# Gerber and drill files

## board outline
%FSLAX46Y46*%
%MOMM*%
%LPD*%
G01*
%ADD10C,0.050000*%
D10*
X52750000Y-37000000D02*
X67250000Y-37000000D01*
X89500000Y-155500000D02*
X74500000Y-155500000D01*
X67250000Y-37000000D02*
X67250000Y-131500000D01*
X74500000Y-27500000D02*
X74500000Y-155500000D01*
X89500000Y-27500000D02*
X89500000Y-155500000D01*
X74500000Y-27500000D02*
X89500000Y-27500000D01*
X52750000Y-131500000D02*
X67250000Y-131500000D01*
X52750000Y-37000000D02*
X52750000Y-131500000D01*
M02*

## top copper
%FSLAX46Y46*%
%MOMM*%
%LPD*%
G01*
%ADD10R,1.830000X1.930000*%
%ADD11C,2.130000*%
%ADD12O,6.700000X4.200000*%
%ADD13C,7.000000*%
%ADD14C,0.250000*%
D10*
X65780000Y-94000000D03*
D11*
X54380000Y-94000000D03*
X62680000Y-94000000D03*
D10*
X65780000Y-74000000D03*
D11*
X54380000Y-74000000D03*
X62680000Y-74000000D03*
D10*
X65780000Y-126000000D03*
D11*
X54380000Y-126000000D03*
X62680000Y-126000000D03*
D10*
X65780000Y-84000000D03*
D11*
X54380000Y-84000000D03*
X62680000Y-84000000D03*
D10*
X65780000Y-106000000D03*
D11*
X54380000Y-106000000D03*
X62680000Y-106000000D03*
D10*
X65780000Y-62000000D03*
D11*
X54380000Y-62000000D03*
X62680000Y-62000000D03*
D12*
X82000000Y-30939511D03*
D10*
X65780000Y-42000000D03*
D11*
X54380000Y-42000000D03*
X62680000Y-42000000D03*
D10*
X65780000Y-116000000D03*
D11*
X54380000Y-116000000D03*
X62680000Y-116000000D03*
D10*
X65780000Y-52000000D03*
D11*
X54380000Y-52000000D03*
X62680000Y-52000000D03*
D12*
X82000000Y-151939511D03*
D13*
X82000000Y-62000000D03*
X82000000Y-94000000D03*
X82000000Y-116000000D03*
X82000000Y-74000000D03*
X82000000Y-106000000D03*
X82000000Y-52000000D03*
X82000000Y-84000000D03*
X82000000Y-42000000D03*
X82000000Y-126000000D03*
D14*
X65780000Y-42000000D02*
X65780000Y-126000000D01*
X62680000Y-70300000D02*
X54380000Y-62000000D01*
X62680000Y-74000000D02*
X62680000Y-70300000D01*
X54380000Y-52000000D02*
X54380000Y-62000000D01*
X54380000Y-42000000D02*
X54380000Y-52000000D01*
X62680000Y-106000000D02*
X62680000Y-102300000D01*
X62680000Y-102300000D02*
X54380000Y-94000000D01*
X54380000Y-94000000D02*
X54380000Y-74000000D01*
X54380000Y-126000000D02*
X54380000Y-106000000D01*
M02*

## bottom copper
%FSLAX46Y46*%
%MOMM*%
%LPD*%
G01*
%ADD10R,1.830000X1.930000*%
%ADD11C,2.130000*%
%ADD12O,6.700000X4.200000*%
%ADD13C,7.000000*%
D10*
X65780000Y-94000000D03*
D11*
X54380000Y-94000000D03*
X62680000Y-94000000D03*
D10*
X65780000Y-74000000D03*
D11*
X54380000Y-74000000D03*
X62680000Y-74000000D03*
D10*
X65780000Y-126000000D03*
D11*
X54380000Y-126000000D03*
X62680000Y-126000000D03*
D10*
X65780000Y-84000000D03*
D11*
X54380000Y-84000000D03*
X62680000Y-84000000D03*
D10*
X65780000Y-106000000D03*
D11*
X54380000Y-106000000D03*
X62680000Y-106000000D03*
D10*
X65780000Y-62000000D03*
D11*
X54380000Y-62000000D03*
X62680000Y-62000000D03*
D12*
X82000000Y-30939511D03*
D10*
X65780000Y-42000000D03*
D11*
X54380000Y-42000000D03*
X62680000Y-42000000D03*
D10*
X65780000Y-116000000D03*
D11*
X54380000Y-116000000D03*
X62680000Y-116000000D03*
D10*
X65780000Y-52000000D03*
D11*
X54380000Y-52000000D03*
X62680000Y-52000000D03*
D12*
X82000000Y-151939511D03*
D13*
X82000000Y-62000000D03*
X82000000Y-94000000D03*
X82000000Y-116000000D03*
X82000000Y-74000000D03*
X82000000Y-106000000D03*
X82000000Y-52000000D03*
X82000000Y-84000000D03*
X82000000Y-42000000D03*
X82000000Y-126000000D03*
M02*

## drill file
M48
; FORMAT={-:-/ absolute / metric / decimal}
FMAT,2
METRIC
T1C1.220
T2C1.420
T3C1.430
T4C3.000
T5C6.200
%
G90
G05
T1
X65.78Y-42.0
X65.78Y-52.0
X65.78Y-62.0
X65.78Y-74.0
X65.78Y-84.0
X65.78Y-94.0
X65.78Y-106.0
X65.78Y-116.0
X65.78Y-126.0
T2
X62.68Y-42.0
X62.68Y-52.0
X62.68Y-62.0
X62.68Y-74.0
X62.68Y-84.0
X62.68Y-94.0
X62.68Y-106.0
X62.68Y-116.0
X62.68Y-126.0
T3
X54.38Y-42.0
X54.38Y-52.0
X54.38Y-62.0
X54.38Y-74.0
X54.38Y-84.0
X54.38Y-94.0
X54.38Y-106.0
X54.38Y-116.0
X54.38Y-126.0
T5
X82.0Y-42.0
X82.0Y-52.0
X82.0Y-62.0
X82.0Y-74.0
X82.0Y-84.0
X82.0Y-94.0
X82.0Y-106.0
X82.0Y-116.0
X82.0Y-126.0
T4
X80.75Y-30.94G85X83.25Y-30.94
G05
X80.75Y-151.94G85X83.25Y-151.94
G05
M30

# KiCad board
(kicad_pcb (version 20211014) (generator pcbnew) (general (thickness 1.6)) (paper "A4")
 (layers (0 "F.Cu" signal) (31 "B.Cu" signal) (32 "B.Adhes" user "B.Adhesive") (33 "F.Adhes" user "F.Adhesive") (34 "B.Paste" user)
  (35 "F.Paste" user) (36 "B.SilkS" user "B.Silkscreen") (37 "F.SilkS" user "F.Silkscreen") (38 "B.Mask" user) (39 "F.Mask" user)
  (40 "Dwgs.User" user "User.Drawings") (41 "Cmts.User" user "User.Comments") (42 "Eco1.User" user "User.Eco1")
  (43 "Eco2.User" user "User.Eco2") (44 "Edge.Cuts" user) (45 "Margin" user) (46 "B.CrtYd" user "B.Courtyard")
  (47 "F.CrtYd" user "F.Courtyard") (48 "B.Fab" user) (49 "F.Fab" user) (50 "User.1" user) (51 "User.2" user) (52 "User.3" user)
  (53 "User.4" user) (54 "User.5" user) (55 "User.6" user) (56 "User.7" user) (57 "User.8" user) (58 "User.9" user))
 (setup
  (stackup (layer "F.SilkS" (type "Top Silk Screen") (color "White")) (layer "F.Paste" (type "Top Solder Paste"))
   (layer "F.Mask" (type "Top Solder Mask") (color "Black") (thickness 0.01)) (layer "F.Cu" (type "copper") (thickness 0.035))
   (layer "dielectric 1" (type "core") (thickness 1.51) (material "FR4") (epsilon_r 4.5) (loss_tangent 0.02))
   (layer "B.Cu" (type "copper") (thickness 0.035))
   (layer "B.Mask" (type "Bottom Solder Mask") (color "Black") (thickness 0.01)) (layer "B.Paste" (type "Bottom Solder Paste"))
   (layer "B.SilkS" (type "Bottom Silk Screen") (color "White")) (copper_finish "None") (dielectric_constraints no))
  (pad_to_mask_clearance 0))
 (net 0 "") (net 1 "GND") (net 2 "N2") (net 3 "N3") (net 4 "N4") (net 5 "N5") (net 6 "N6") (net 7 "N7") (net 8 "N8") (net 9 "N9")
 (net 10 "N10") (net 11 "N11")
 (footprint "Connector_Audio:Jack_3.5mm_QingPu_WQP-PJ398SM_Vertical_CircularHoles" (layer "F.Cu") (at 65.78 94 -90)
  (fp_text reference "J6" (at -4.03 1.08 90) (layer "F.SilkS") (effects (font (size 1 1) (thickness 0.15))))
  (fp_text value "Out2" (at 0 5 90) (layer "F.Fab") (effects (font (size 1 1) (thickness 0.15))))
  (pad "S" thru_hole rect locked (at 0 0 90) (size 1.93 1.83) (drill 1.22) (layers *.Cu *.Mask) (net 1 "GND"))
  (pad "T" thru_hole circle locked (at 0 11.4 90) (size 2.13 2.13) (drill 1.43) (layers *.Cu *.Mask) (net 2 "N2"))
  (pad "TN" thru_hole circle locked (at 0 3.1 90) (size 2.13 2.13) (drill 1.42) (layers *.Cu *.Mask) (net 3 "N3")))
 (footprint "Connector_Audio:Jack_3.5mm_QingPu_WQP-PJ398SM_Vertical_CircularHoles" (layer "F.Cu") (at 65.78 74 -90)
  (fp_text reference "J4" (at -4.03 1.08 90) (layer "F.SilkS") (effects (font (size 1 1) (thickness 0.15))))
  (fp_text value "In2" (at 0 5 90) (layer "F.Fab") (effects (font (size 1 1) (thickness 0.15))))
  (pad "S" thru_hole rect locked (at 0 0 90) (size 1.93 1.83) (drill 1.22) (layers *.Cu *.Mask) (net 1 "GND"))
  (pad "T" thru_hole circle locked (at 0 11.4 90) (size 2.13 2.13) (drill 1.43) (layers *.Cu *.Mask) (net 2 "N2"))
  (pad "TN" thru_hole circle locked (at 0 3.1 90) (size 2.13 2.13) (drill 1.42) (layers *.Cu *.Mask) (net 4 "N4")))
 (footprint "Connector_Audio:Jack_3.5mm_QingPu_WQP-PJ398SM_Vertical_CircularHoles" (layer "F.Cu") (at 65.78 126 -90)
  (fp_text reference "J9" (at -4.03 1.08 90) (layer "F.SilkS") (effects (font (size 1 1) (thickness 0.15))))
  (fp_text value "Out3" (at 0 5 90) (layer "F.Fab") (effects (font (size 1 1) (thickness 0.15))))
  (pad "S" thru_hole rect locked (at 0 0 90) (size 1.93 1.83) (drill 1.22) (layers *.Cu *.Mask) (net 1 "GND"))
  (pad "T" thru_hole circle locked (at 0 11.4 90) (size 2.13 2.13) (drill 1.43) (layers *.Cu *.Mask) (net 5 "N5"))
  (pad "TN" thru_hole circle locked (at 0 3.1 90) (size 2.13 2.13) (drill 1.42) (layers *.Cu *.Mask) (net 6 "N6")))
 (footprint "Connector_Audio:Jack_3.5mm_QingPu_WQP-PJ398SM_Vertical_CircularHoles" (layer "F.Cu") (at 65.78 84 -90)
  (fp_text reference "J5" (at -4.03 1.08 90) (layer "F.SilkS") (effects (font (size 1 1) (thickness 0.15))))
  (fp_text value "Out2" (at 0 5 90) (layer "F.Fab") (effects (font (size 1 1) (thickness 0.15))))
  (pad "S" thru_hole rect locked (at 0 0 90) (size 1.93 1.83) (drill 1.22) (layers *.Cu *.Mask) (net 1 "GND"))
  (pad "T" thru_hole circle locked (at 0 11.4 90) (size 2.13 2.13) (drill 1.43) (layers *.Cu *.Mask) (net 2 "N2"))
  (pad "TN" thru_hole circle locked (at 0 3.1 90) (size 2.13 2.13) (drill 1.42) (layers *.Cu *.Mask) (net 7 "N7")))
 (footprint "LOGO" (layer "F.Cu") (at 82 136.5)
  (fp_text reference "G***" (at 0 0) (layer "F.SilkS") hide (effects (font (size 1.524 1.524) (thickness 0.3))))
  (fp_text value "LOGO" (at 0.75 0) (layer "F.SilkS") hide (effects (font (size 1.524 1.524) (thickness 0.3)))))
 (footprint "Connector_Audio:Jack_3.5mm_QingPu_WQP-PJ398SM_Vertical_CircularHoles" (layer "F.Cu") (at 65.78 106 -90)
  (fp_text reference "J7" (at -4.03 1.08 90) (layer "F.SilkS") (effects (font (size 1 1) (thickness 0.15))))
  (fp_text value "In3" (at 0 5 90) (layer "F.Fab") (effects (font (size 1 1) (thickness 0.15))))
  (pad "S" thru_hole rect locked (at 0 0 90) (size 1.93 1.83) (drill 1.22) (layers *.Cu *.Mask) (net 1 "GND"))
  (pad "T" thru_hole circle locked (at 0 11.4 90) (size 2.13 2.13) (drill 1.43) (layers *.Cu *.Mask) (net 5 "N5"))
  (pad "TN" thru_hole circle locked (at 0 3.1 90) (size 2.13 2.13) (drill 1.42) (layers *.Cu *.Mask) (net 2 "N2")))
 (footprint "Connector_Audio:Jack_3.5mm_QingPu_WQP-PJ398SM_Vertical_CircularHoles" (layer "F.Cu") (at 65.78 62 -90)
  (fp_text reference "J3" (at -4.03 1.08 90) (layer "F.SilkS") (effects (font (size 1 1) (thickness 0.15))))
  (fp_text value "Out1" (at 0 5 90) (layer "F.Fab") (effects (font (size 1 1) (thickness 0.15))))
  (pad "S" thru_hole rect locked (at 0 0 90) (size 1.93 1.83) (drill 1.22) (layers *.Cu *.Mask) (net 1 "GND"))
  (pad "T" thru_hole circle locked (at 0 11.4 90) (size 2.13 2.13) (drill 1.43) (layers *.Cu *.Mask) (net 4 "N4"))
  (pad "TN" thru_hole circle locked (at 0 3.1 90) (size 2.13 2.13) (drill 1.42) (layers *.Cu *.Mask) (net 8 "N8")))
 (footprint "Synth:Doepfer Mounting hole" (layer "F.Cu") (at 82 30.939511)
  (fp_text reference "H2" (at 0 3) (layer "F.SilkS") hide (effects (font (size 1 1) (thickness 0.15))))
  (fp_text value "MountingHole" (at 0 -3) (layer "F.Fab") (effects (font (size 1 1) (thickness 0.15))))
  (pad "1" thru_hole oval locked (at 0 0) (size 6.7 4.2) (drill oval 5.5 3) (layers *.Cu *.Mask)))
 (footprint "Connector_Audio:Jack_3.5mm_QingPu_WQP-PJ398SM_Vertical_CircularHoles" (layer "F.Cu") (at 65.78 42 -90)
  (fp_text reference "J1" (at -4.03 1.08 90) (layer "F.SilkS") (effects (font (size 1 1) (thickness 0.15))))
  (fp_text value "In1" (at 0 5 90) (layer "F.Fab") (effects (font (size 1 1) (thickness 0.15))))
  (pad "S" thru_hole rect locked (at 0 0 90) (size 1.93 1.83) (drill 1.22) (layers *.Cu *.Mask) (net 1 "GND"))
  (pad "T" thru_hole circle locked (at 0 11.4 90) (size 2.13 2.13) (drill 1.43) (layers *.Cu *.Mask) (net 4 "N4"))
  (pad "TN" thru_hole circle locked (at 0 3.1 90) (size 2.13 2.13) (drill 1.42) (layers *.Cu *.Mask) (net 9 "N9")))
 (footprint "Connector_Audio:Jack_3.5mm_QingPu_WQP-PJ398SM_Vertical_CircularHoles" (layer "F.Cu") (at 65.78 116 -90)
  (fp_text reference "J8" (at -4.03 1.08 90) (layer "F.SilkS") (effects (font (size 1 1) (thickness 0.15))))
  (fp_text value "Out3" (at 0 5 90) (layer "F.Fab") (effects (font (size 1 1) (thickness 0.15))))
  (pad "S" thru_hole rect locked (at 0 0 90) (size 1.93 1.83) (drill 1.22) (layers *.Cu *.Mask) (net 1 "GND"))
  (pad "T" thru_hole circle locked (at 0 11.4 90) (size 2.13 2.13) (drill 1.43) (layers *.Cu *.Mask) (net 5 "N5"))
  (pad "TN" thru_hole circle locked (at 0 3.1 90) (size 2.13 2.13) (drill 1.42) (layers *.Cu *.Mask) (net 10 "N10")))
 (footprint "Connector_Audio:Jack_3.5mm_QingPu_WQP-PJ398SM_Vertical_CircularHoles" (layer "F.Cu") (at 65.78 52 -90)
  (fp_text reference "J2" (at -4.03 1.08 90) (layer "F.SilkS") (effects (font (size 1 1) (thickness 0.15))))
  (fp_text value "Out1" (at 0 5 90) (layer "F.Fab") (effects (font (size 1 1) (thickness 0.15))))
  (pad "S" thru_hole rect locked (at 0 0 90) (size 1.93 1.83) (drill 1.22) (layers *.Cu *.Mask) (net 1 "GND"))
  (pad "T" thru_hole circle locked (at 0 11.4 90) (size 2.13 2.13) (drill 1.43) (layers *.Cu *.Mask) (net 4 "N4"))
  (pad "TN" thru_hole circle locked (at 0 3.1 90) (size 2.13 2.13) (drill 1.42) (layers *.Cu *.Mask) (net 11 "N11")))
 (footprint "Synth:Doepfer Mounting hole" (layer "F.Cu") (at 82 151.939511)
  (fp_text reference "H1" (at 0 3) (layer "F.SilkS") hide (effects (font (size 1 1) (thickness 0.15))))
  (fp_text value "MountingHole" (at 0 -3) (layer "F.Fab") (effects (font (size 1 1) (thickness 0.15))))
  (pad "1" thru_hole oval locked (at 0 0) (size 6.7 4.2) (drill oval 5.5 3) (layers *.Cu *.Mask)))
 (gr_line (start 52.75 37) (end 67.25 37) (layer "Edge.Cuts") (width 0.05))
 (gr_line (start 89.5 155.5) (end 74.5 155.5) (layer "Edge.Cuts") (width 0.05))
 (gr_line (start 67.25 37) (end 67.25 131.5) (layer "Edge.Cuts") (width 0.05))
 (gr_line (start 74.5 27.5) (end 74.5 155.5) (layer "Edge.Cuts") (width 0.05))
 (gr_line (start 89.5 27.5) (end 89.5 155.5) (layer "Edge.Cuts") (width 0.05))
 (gr_line (start 74.5 27.5) (end 89.5 27.5) (layer "Edge.Cuts") (width 0.05))
 (gr_line (start 52.75 131.5) (end 67.25 131.5) (layer "Edge.Cuts") (width 0.05))
 (gr_line (start 52.75 37) (end 52.75 131.5) (layer "Edge.Cuts") (width 0.05))
 (via (at 82 62) (size 7) (drill 6.2) (layers "F.Cu" "B.Cu") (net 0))
 (via (at 82 94) (size 7) (drill 6.2) (layers "F.Cu" "B.Cu") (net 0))
 (via (at 82 116) (size 7) (drill 6.2) (layers "F.Cu" "B.Cu") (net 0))
 (via (at 82 74) (size 7) (drill 6.2) (layers "F.Cu" "B.Cu") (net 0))
 (via (at 82 106) (size 7) (drill 6.2) (layers "F.Cu" "B.Cu") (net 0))
 (via (at 82 52) (size 7) (drill 6.2) (layers "F.Cu" "B.Cu") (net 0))
 (via (at 82 84) (size 7) (drill 6.2) (layers "F.Cu" "B.Cu") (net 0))
 (via (at 82 42) (size 7) (drill 6.2) (layers "F.Cu" "B.Cu") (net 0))
 (via (at 82 126) (size 7) (drill 6.2) (layers "F.Cu" "B.Cu") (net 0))
 (segment (start 65.78 42) (end 65.78 126) (width 0.25) (layer "F.Cu") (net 1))
 (segment (start 62.68 70.3) (end 54.38 62) (width 0.25) (layer "F.Cu") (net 4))
 (segment (start 62.68 74) (end 62.68 70.3) (width 0.25) (layer "F.Cu") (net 4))
 (segment (start 54.38 52) (end 54.38 62) (width 0.25) (layer "F.Cu") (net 4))
 (segment (start 54.38 42) (end 54.38 52) (width 0.25) (layer "F.Cu") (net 4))
 (segment (start 62.68 106) (end 62.68 102.3) (width 0.25) (layer "F.Cu") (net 2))
 (segment (start 62.68 102.3) (end 54.38 94) (width 0.25) (layer "F.Cu") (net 2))
 (segment (start 54.38 94) (end 54.38 74) (width 0.25) (layer "F.Cu") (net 2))
 (segment (start 54.38 126) (end 54.38 106) (width 0.25) (layer "F.Cu") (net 5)))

